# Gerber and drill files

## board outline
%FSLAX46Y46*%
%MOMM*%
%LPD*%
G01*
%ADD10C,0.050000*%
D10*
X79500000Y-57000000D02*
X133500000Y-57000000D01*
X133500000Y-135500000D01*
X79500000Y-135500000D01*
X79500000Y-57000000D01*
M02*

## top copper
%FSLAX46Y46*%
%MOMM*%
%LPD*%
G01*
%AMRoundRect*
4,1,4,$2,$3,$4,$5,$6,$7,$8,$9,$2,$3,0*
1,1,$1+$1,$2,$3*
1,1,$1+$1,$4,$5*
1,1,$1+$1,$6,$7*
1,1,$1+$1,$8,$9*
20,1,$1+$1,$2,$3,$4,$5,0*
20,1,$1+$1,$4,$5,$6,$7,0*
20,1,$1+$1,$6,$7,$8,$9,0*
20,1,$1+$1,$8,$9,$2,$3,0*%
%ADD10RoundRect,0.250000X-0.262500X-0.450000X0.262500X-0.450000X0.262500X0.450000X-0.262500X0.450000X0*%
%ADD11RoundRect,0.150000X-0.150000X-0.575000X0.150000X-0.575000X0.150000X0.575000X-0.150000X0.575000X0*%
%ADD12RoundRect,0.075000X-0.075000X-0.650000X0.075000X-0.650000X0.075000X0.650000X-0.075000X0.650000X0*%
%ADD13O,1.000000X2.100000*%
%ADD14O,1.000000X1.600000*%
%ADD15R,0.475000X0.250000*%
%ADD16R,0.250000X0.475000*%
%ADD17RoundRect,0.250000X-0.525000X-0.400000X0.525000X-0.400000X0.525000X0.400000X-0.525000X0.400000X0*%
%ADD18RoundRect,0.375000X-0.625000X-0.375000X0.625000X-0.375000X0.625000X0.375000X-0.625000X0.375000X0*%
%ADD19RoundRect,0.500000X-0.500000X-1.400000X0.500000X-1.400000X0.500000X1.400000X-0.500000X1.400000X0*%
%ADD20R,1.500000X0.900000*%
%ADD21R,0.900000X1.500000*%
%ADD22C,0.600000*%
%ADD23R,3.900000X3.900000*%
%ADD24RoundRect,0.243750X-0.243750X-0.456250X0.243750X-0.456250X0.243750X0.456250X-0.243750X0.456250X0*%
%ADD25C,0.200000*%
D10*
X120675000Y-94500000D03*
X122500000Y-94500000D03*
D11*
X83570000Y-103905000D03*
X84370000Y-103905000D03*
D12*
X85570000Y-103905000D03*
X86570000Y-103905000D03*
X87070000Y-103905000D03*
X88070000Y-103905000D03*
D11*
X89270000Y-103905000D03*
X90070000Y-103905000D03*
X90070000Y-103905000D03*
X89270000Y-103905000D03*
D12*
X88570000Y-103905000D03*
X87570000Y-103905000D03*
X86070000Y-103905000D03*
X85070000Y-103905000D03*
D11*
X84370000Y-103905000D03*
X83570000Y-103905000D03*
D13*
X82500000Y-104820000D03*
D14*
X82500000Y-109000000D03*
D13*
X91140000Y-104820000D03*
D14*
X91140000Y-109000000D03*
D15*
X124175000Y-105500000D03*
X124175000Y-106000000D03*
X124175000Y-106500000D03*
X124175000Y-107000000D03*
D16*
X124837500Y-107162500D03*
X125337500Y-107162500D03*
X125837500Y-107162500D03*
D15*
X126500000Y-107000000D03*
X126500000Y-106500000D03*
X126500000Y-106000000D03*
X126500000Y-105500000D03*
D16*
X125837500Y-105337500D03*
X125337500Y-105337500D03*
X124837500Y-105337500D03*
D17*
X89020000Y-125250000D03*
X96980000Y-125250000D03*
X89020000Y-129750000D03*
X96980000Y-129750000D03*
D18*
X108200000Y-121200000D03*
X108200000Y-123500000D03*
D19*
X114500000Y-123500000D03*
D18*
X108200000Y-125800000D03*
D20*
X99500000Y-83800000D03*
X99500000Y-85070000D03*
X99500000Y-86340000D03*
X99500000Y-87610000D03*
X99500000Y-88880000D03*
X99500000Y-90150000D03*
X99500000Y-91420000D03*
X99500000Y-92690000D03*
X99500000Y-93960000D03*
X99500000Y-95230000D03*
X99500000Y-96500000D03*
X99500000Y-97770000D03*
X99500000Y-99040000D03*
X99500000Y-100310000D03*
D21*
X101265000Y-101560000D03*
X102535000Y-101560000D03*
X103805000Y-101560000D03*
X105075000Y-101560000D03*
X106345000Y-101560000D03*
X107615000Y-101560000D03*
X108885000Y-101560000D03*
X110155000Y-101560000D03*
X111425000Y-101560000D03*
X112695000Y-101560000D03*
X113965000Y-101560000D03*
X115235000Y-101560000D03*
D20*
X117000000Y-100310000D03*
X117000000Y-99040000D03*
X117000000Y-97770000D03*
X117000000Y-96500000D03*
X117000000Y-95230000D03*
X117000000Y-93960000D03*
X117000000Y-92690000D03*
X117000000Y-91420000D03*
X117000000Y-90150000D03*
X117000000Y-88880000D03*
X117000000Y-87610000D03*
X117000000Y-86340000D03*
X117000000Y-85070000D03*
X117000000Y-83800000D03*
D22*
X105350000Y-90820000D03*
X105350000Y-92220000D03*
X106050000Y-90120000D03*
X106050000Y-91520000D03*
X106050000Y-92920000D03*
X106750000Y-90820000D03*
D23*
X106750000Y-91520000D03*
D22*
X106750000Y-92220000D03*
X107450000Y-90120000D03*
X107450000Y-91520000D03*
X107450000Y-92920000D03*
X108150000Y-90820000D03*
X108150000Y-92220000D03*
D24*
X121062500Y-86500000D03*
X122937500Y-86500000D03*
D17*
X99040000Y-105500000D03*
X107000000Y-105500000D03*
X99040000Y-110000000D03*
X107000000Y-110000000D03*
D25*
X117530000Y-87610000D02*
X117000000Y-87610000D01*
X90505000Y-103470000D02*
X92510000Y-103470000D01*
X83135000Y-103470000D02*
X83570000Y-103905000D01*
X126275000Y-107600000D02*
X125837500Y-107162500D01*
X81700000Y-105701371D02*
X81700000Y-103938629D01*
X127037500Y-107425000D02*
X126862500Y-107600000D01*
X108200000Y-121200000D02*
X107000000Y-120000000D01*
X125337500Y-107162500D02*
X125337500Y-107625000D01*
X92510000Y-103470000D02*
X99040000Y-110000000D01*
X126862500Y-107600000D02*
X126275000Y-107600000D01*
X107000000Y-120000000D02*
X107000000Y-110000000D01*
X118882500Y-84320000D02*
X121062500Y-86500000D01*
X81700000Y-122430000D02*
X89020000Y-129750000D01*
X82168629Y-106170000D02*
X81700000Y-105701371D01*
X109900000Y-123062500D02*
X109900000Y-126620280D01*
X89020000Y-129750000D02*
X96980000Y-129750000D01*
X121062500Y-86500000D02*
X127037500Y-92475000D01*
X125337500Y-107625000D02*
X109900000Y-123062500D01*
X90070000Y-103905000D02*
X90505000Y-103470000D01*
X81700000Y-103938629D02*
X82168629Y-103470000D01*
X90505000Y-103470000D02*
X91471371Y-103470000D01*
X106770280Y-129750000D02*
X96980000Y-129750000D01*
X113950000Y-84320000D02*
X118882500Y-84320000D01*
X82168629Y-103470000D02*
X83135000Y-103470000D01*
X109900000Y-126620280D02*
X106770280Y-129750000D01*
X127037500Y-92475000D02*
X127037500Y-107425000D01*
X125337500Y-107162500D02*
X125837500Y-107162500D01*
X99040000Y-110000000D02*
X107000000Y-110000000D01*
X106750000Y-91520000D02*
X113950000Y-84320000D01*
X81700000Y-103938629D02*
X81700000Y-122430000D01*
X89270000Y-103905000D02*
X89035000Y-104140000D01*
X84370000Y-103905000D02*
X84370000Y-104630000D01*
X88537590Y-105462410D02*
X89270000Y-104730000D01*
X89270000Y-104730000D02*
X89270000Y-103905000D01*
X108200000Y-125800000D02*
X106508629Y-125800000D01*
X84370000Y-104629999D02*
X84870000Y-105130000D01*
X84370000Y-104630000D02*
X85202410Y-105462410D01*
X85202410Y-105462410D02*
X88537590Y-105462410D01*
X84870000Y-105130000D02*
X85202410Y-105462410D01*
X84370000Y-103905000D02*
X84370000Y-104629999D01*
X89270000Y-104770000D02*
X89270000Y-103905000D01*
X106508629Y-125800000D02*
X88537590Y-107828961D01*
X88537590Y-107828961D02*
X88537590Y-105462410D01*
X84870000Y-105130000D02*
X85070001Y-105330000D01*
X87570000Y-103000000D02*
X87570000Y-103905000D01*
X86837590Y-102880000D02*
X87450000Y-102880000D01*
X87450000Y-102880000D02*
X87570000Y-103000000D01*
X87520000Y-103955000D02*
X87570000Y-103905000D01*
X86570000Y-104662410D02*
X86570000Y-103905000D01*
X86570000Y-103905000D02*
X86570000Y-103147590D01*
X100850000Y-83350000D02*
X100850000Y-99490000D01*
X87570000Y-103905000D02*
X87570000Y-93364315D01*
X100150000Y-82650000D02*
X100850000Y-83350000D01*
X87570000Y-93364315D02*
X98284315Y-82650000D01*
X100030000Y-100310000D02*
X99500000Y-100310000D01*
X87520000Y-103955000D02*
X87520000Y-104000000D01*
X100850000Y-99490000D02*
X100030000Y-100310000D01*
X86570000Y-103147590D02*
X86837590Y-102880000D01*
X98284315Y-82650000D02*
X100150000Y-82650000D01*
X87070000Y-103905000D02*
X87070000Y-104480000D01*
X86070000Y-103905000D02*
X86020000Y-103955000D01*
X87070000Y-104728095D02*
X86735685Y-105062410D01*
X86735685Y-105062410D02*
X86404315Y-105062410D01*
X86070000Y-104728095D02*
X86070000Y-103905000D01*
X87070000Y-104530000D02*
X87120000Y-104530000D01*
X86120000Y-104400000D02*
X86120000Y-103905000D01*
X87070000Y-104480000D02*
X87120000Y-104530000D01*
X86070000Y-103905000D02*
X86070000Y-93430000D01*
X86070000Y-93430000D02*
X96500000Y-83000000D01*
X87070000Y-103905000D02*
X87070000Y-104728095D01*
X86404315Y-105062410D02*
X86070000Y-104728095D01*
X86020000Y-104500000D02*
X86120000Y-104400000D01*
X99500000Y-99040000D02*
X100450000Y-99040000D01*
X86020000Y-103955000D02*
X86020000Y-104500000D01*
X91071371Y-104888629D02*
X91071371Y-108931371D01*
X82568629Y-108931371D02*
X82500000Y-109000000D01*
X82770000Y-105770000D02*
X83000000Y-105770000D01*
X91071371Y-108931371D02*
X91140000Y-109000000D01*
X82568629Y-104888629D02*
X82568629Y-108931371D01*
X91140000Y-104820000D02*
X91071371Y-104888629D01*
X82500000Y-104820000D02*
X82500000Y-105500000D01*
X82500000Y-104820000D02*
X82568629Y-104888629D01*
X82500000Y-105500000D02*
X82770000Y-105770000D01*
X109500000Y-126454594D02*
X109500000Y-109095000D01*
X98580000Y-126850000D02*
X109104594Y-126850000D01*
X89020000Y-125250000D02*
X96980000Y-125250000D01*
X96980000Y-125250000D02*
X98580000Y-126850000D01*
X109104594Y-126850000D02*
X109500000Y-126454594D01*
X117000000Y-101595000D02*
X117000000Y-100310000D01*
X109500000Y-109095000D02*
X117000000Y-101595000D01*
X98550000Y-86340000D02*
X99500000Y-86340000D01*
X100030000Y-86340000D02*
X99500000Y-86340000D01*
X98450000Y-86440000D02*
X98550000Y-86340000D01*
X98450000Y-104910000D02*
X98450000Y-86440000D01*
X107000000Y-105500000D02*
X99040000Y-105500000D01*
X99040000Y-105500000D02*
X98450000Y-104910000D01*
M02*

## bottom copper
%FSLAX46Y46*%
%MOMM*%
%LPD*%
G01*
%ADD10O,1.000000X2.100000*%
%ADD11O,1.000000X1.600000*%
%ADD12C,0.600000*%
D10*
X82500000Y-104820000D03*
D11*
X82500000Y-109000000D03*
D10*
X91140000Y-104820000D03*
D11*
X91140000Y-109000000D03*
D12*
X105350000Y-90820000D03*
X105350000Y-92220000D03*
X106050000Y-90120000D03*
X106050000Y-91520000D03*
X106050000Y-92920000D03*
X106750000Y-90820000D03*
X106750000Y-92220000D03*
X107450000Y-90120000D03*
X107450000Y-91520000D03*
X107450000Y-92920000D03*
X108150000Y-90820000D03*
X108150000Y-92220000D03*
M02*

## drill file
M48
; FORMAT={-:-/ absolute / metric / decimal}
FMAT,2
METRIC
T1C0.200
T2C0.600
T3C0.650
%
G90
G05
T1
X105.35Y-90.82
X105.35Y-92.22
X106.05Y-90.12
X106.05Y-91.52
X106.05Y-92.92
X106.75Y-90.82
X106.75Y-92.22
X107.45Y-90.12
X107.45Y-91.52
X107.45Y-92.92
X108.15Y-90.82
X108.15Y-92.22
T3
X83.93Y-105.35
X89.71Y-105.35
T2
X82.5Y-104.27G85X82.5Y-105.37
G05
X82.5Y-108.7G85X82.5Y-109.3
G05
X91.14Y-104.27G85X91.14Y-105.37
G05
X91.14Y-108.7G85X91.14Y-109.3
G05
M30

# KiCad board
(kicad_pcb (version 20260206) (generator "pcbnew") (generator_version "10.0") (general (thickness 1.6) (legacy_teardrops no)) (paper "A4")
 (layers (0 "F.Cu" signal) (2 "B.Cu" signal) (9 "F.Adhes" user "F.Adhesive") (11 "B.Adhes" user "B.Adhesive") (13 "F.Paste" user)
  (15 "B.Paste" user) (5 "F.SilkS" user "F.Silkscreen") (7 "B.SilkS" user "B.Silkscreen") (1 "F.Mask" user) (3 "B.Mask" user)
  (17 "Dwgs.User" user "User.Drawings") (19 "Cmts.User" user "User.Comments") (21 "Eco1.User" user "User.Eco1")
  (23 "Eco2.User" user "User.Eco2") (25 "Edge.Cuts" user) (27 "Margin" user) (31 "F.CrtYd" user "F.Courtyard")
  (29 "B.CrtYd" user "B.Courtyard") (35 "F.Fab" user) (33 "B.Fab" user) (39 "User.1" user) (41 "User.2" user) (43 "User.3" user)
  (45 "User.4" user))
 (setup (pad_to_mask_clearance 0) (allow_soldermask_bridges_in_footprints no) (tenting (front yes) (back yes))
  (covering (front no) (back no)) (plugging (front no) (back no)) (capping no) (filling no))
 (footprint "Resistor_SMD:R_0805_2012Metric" (layer "F.Cu") (at 121.5875 94.5)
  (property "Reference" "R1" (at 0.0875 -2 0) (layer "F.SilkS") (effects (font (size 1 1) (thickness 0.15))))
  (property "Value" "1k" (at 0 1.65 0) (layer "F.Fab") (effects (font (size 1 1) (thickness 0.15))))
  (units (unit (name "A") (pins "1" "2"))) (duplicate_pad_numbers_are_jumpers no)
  (pad "1" smd roundrect (at -0.9125 0) (size 1.025 1.4) (layers "F.Cu" "F.Mask" "F.Paste") (roundrect_rratio 0.243902) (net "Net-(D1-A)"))
  (pad "2" smd roundrect (at 0.9125 0) (size 1.025 1.4) (layers "F.Cu" "F.Mask" "F.Paste") (roundrect_rratio 0.243902) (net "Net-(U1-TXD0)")))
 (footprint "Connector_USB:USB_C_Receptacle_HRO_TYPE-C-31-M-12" (layer "F.Cu") (at 86.82 107.95)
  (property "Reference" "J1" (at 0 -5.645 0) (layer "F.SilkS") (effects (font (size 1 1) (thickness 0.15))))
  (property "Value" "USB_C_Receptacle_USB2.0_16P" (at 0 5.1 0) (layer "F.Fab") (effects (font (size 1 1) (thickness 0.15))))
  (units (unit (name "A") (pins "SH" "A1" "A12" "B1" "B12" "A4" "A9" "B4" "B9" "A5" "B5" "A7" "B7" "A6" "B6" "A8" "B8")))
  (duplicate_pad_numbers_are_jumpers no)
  (pad "" np_thru_hole circle (at -2.89 -2.6) (size 0.65 0.65) (drill 0.65) (layers "*.Cu" "*.Mask"))
  (pad "" np_thru_hole circle (at 2.89 -2.6) (size 0.65 0.65) (drill 0.65) (layers "*.Cu" "*.Mask"))
  (pad "A1" smd roundrect (at -3.25 -4.045) (size 0.6 1.45) (layers "F.Cu" "F.Mask" "F.Paste") (roundrect_rratio 0.25) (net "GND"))
  (pad "A4" smd roundrect (at -2.45 -4.045) (size 0.6 1.45) (layers "F.Cu" "F.Mask" "F.Paste") (roundrect_rratio 0.25) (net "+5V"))
  (pad "A5" smd roundrect (at -1.25 -4.045) (size 0.3 1.45) (layers "F.Cu" "F.Mask" "F.Paste") (roundrect_rratio 0.25)
   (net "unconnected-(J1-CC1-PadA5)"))
  (pad "A6" smd roundrect (at -0.25 -4.045) (size 0.3 1.45) (layers "F.Cu" "F.Mask" "F.Paste") (roundrect_rratio 0.25)
   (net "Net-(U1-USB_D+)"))
  (pad "A7" smd roundrect (at 0.25 -4.045) (size 0.3 1.45) (layers "F.Cu" "F.Mask" "F.Paste") (roundrect_rratio 0.25)
   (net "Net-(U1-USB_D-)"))
  (pad "A8" smd roundrect (at 1.25 -4.045) (size 0.3 1.45) (layers "F.Cu" "F.Mask" "F.Paste") (roundrect_rratio 0.25)
   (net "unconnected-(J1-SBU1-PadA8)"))
  (pad "A9" smd roundrect (at 2.45 -4.045) (size 0.6 1.45) (layers "F.Cu" "F.Mask" "F.Paste") (roundrect_rratio 0.25) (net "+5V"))
  (pad "A12" smd roundrect (at 3.25 -4.045) (size 0.6 1.45) (layers "F.Cu" "F.Mask" "F.Paste") (roundrect_rratio 0.25) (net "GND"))
  (pad "B1" smd roundrect (at 3.25 -4.045) (size 0.6 1.45) (layers "F.Cu" "F.Mask" "F.Paste") (roundrect_rratio 0.25) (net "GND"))
  (pad "B4" smd roundrect (at 2.45 -4.045) (size 0.6 1.45) (layers "F.Cu" "F.Mask" "F.Paste") (roundrect_rratio 0.25) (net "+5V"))
  (pad "B5" smd roundrect (at 1.75 -4.045) (size 0.3 1.45) (layers "F.Cu" "F.Mask" "F.Paste") (roundrect_rratio 0.25)
   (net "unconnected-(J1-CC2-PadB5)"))
  (pad "B6" smd roundrect (at 0.75 -4.045) (size 0.3 1.45) (layers "F.Cu" "F.Mask" "F.Paste") (roundrect_rratio 0.25)
   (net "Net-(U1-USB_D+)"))
  (pad "B7" smd roundrect (at -0.75 -4.045) (size 0.3 1.45) (layers "F.Cu" "F.Mask" "F.Paste") (roundrect_rratio 0.25)
   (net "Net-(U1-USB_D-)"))
  (pad "B8" smd roundrect (at -1.75 -4.045) (size 0.3 1.45) (layers "F.Cu" "F.Mask" "F.Paste") (roundrect_rratio 0.25)
   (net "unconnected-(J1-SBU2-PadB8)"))
  (pad "B9" smd roundrect (at -2.45 -4.045) (size 0.6 1.45) (layers "F.Cu" "F.Mask" "F.Paste") (roundrect_rratio 0.25) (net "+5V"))
  (pad "B12" smd roundrect (at -3.25 -4.045) (size 0.6 1.45) (layers "F.Cu" "F.Mask" "F.Paste") (roundrect_rratio 0.25) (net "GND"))
  (pad "SH" thru_hole oval (at -4.32 -3.13) (size 1 2.1) (drill oval 0.6 1.7) (layers "*.Cu" "*.Mask") (remove_unused_layers no)
   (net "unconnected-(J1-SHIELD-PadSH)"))
  (pad "SH" thru_hole oval (at -4.32 1.05) (size 1 1.6) (drill oval 0.6 1.2) (layers "*.Cu" "*.Mask") (remove_unused_layers no)
   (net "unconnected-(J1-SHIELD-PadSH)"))
  (pad "SH" thru_hole oval (at 4.32 -3.13) (size 1 2.1) (drill oval 0.6 1.7) (layers "*.Cu" "*.Mask") (remove_unused_layers no)
   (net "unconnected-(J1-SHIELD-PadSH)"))
  (pad "SH" thru_hole oval (at 4.32 1.05) (size 1 1.6) (drill oval 0.6 1.2) (layers "*.Cu" "*.Mask") (remove_unused_layers no)
   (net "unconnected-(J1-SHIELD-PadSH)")))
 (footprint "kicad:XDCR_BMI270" (layer "F.Cu") (at 125.3375 106.25)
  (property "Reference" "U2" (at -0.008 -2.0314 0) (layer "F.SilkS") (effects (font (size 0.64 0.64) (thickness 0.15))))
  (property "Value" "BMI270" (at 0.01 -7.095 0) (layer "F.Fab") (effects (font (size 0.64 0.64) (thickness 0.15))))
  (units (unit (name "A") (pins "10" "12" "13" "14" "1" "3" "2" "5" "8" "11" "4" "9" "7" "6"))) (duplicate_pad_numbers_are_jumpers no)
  (pad "1" smd rect (at -1.1625 -0.75) (size 0.475 0.25) (layers "F.Cu" "F.Mask" "F.Paste") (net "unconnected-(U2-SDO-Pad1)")
   (solder_mask_margin 0.102))
  (pad "2" smd rect (at -1.1625 -0.25) (size 0.475 0.25) (layers "F.Cu" "F.Mask" "F.Paste") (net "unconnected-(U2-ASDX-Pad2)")
   (solder_mask_margin 0.102))
  (pad "3" smd rect (at -1.1625 0.25) (size 0.475 0.25) (layers "F.Cu" "F.Mask" "F.Paste") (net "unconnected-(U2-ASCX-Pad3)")
   (solder_mask_margin 0.102))
  (pad "4" smd rect (at -1.1625 0.75) (size 0.475 0.25) (layers "F.Cu" "F.Mask" "F.Paste") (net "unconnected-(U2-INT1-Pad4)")
   (solder_mask_margin 0.102))
  (pad "5" smd rect (at -0.5 0.9125) (size 0.25 0.475) (layers "F.Cu" "F.Mask" "F.Paste") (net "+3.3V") (solder_mask_margin 0.102))
  (pad "6" smd rect (at 0 0.9125) (size 0.25 0.475) (layers "F.Cu" "F.Mask" "F.Paste") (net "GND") (solder_mask_margin 0.102))
  (pad "7" smd rect (at 0.5 0.9125) (size 0.25 0.475) (layers "F.Cu" "F.Mask" "F.Paste") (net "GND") (solder_mask_margin 0.102))
  (pad "8" smd rect (at 1.1625 0.75) (size 0.475 0.25) (layers "F.Cu" "F.Mask" "F.Paste") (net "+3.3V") (solder_mask_margin 0.102))
  (pad "9" smd rect (at 1.1625 0.25) (size 0.475 0.25) (layers "F.Cu" "F.Mask" "F.Paste") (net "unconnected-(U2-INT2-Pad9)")
   (solder_mask_margin 0.102))
  (pad "10" smd rect (at 1.1625 -0.25) (size 0.475 0.25) (layers "F.Cu" "F.Mask" "F.Paste") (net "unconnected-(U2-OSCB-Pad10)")
   (solder_mask_margin 0.102))
  (pad "11" smd rect (at 1.1625 -0.75) (size 0.475 0.25) (layers "F.Cu" "F.Mask" "F.Paste") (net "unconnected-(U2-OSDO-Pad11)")
   (solder_mask_margin 0.102))
  (pad "12" smd rect (at 0.5 -0.9125) (size 0.25 0.475) (layers "F.Cu" "F.Mask" "F.Paste") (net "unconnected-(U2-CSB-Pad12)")
   (solder_mask_margin 0.102))
  (pad "13" smd rect (at 0 -0.9125) (size 0.25 0.475) (layers "F.Cu" "F.Mask" "F.Paste") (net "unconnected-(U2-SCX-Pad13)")
   (solder_mask_margin 0.102))
  (pad "14" smd rect (at -0.5 -0.9125) (size 0.25 0.475) (layers "F.Cu" "F.Mask" "F.Paste") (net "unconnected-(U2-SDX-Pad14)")
   (solder_mask_margin 0.102)))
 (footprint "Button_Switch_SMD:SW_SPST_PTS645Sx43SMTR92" (layer "F.Cu") (at 93 127.5)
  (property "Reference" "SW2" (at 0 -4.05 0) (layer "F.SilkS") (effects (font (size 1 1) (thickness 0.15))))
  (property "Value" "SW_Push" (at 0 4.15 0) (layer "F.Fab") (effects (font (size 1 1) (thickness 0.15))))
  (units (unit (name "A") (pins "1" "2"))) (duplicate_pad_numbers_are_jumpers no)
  (pad "1" smd roundrect (at -3.98 -2.25) (size 1.55 1.3) (layers "F.Cu" "F.Mask" "F.Paste") (roundrect_rratio 0.1923076923)
   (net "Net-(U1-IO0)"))
  (pad "1" smd roundrect (at 3.98 -2.25) (size 1.55 1.3) (layers "F.Cu" "F.Mask" "F.Paste") (roundrect_rratio 0.1923076923)
   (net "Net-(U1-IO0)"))
  (pad "2" smd roundrect (at -3.98 2.25) (size 1.55 1.3) (layers "F.Cu" "F.Mask" "F.Paste") (roundrect_rratio 0.1923076923) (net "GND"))
  (pad "2" smd roundrect (at 3.98 2.25) (size 1.55 1.3) (layers "F.Cu" "F.Mask" "F.Paste") (roundrect_rratio 0.1923076923) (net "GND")))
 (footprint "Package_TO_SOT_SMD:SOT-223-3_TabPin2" (layer "F.Cu") (at 111.35 123.5)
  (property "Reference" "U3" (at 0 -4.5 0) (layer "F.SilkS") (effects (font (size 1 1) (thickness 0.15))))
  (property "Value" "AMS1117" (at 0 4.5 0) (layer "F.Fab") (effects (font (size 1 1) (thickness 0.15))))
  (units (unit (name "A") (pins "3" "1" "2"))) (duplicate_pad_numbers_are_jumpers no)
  (pad "1" smd roundrect (at -3.15 -2.3) (size 2 1.5) (layers "F.Cu" "F.Mask" "F.Paste") (roundrect_rratio 0.25) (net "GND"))
  (pad "2" smd roundrect (at -3.15 0) (size 2 1.5) (layers "F.Cu" "F.Mask" "F.Paste") (roundrect_rratio 0.25) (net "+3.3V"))
  (pad "2" smd roundrect (at 3.15 0) (size 2 3.8) (layers "F.Cu" "F.Mask" "F.Paste") (roundrect_rratio 0.25) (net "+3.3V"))
  (pad "3" smd roundrect (at -3.15 2.3) (size 2 1.5) (layers "F.Cu" "F.Mask" "F.Paste") (roundrect_rratio 0.25) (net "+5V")))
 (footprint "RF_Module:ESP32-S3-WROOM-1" (layer "F.Cu") (at 108.25 89.06)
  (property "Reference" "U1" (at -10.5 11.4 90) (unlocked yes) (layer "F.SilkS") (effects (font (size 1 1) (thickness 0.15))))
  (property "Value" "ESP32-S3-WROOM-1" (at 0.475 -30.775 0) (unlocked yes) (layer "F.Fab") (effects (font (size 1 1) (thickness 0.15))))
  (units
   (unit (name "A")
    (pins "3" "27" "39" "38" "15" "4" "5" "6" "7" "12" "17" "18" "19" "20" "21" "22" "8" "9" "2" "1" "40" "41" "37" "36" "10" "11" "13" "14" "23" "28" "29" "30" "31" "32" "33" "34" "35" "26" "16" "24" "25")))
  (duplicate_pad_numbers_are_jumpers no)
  (pad "" smd rect (at -2.9 1.06) (size 0.9 0.9) (layers "F.Paste"))
  (pad "" smd rect (at -2.9 2.46 270) (size 0.9 0.9) (layers "F.Paste"))
  (pad "" smd rect (at -2.9 3.86) (size 0.9 0.9) (layers "F.Paste"))
  (pad "" smd rect (at -1.5 1.06 270) (size 0.9 0.9) (layers "F.Paste"))
  (pad "" smd rect (at -1.5 2.46 270) (size 0.9 0.9) (layers "F.Paste"))
  (pad "" smd rect (at -1.5 3.86 270) (size 0.9 0.9) (layers "F.Paste"))
  (pad "" smd rect (at -0.1 1.06 270) (size 0.9 0.9) (layers "F.Paste"))
  (pad "" smd rect (at -0.1 2.46 270) (size 0.9 0.9) (layers "F.Paste"))
  (pad "" smd rect (at -0.1 3.86 270) (size 0.9 0.9) (layers "F.Paste"))
  (pad "1" smd rect (at -8.75 -5.26) (size 1.5 0.9) (layers "F.Cu" "F.Mask" "F.Paste") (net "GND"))
  (pad "2" smd rect (at -8.75 -3.99) (size 1.5 0.9) (layers "F.Cu" "F.Mask" "F.Paste") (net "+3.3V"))
  (pad "3" smd rect (at -8.75 -2.72) (size 1.5 0.9) (layers "F.Cu" "F.Mask" "F.Paste") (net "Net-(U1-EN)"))
  (pad "4" smd rect (at -8.75 -1.45) (size 1.5 0.9) (layers "F.Cu" "F.Mask" "F.Paste") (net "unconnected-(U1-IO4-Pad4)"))
  (pad "5" smd rect (at -8.75 -0.18) (size 1.5 0.9) (layers "F.Cu" "F.Mask" "F.Paste") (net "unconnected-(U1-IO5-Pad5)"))
  (pad "6" smd rect (at -8.75 1.09) (size 1.5 0.9) (layers "F.Cu" "F.Mask" "F.Paste") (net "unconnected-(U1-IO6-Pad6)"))
  (pad "7" smd rect (at -8.75 2.36) (size 1.5 0.9) (layers "F.Cu" "F.Mask" "F.Paste") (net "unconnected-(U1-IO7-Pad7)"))
  (pad "8" smd rect (at -8.75 3.63) (size 1.5 0.9) (layers "F.Cu" "F.Mask" "F.Paste") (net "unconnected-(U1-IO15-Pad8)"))
  (pad "9" smd rect (at -8.75 4.9) (size 1.5 0.9) (layers "F.Cu" "F.Mask" "F.Paste") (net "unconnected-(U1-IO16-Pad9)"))
  (pad "10" smd rect (at -8.75 6.17) (size 1.5 0.9) (layers "F.Cu" "F.Mask" "F.Paste") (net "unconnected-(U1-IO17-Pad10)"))
  (pad "11" smd rect (at -8.75 7.44) (size 1.5 0.9) (layers "F.Cu" "F.Mask" "F.Paste") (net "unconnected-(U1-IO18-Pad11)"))
  (pad "12" smd rect (at -8.75 8.71) (size 1.5 0.9) (layers "F.Cu" "F.Mask" "F.Paste") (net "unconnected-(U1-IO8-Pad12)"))
  (pad "13" smd rect (at -8.75 9.98) (size 1.5 0.9) (layers "F.Cu" "F.Mask" "F.Paste") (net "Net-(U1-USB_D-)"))
  (pad "14" smd rect (at -8.75 11.25 180) (size 1.5 0.9) (layers "F.Cu" "F.Mask" "F.Paste") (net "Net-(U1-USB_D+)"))
  (pad "15" smd rect (at -6.985 12.5 270) (size 1.5 0.9) (layers "F.Cu" "F.Mask" "F.Paste") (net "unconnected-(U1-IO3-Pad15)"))
  (pad "16" smd rect (at -5.715 12.5 270) (size 1.5 0.9) (layers "F.Cu" "F.Mask" "F.Paste") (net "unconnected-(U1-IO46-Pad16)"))
  (pad "17" smd rect (at -4.445 12.5 270) (size 1.5 0.9) (layers "F.Cu" "F.Mask" "F.Paste") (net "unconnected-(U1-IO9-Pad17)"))
  (pad "18" smd rect (at -3.175 12.5 270) (size 1.5 0.9) (layers "F.Cu" "F.Mask" "F.Paste") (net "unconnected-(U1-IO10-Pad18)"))
  (pad "19" smd rect (at -1.905 12.5 270) (size 1.5 0.9) (layers "F.Cu" "F.Mask" "F.Paste") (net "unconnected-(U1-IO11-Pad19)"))
  (pad "20" smd rect (at -0.635 12.5 270) (size 1.5 0.9) (layers "F.Cu" "F.Mask" "F.Paste") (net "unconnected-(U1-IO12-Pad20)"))
  (pad "21" smd rect (at 0.635 12.5 270) (size 1.5 0.9) (layers "F.Cu" "F.Mask" "F.Paste") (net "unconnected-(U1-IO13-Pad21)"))
  (pad "22" smd rect (at 1.905 12.5 270) (size 1.5 0.9) (layers "F.Cu" "F.Mask" "F.Paste") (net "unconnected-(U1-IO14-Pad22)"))
  (pad "23" smd rect (at 3.175 12.5 270) (size 1.5 0.9) (layers "F.Cu" "F.Mask" "F.Paste") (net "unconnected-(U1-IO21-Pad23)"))
  (pad "24" smd rect (at 4.445 12.5 270) (size 1.5 0.9) (layers "F.Cu" "F.Mask" "F.Paste") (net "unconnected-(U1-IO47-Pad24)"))
  (pad "25" smd rect (at 5.715 12.5 270) (size 1.5 0.9) (layers "F.Cu" "F.Mask" "F.Paste") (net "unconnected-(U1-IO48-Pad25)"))
  (pad "26" smd rect (at 6.985 12.5 270) (size 1.5 0.9) (layers "F.Cu" "F.Mask" "F.Paste") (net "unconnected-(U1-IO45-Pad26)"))
  (pad "27" smd rect (at 8.75 11.25) (size 1.5 0.9) (layers "F.Cu" "F.Mask" "F.Paste") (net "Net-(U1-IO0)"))
  (pad "28" smd rect (at 8.75 9.98) (size 1.5 0.9) (layers "F.Cu" "F.Mask" "F.Paste") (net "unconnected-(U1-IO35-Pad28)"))
  (pad "29" smd rect (at 8.75 8.71) (size 1.5 0.9) (layers "F.Cu" "F.Mask" "F.Paste") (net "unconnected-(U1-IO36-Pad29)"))
  (pad "30" smd rect (at 8.75 7.44) (size 1.5 0.9) (layers "F.Cu" "F.Mask" "F.Paste") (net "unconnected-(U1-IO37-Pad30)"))
  (pad "31" smd rect (at 8.75 6.17) (size 1.5 0.9) (layers "F.Cu" "F.Mask" "F.Paste") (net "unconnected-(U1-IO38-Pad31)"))
  (pad "32" smd rect (at 8.75 4.9) (size 1.5 0.9) (layers "F.Cu" "F.Mask" "F.Paste") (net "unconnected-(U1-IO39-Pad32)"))
  (pad "33" smd rect (at 8.75 3.63) (size 1.5 0.9) (layers "F.Cu" "F.Mask" "F.Paste") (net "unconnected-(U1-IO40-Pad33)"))
  (pad "34" smd rect (at 8.75 2.36) (size 1.5 0.9) (layers "F.Cu" "F.Mask" "F.Paste") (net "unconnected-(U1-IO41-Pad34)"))
  (pad "35" smd rect (at 8.75 1.09) (size 1.5 0.9) (layers "F.Cu" "F.Mask" "F.Paste") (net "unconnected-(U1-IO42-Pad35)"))
  (pad "36" smd rect (at 8.75 -0.18) (size 1.5 0.9) (layers "F.Cu" "F.Mask" "F.Paste") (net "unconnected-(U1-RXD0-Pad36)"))
  (pad "37" smd rect (at 8.75 -1.45) (size 1.5 0.9) (layers "F.Cu" "F.Mask" "F.Paste") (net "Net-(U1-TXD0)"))
  (pad "38" smd rect (at 8.75 -2.72) (size 1.5 0.9) (layers "F.Cu" "F.Mask" "F.Paste") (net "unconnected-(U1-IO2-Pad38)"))
  (pad "39" smd rect (at 8.75 -3.99) (size 1.5 0.9) (layers "F.Cu" "F.Mask" "F.Paste") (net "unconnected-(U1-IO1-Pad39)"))
  (pad "40" smd rect (at 8.75 -5.26) (size 1.5 0.9) (layers "F.Cu" "F.Mask" "F.Paste") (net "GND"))
  (pad "41" thru_hole circle (at -2.9 1.76 90) (size 0.6 0.6) (drill 0.2) (layers "*.Cu" "F.Mask") (remove_unused_layers no) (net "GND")
   (zone_connect 2))
  (pad "41" thru_hole circle (at -2.9 3.16) (size 0.6 0.6) (drill 0.2) (layers "*.Cu" "F.Mask") (remove_unused_layers no) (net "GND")
   (zone_connect 2))
  (pad "41" thru_hole circle (at -2.2 1.06) (size 0.6 0.6) (drill 0.2) (layers "*.Cu" "F.Mask") (remove_unused_layers no) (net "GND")
   (zone_connect 2))
  (pad "41" thru_hole circle (at -2.2 2.46) (size 0.6 0.6) (drill 0.2) (layers "*.Cu" "F.Mask") (remove_unused_layers no) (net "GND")
   (zone_connect 2))
  (pad "41" thru_hole circle (at -2.2 3.86) (size 0.6 0.6) (drill 0.2) (layers "*.Cu" "F.Mask") (remove_unused_layers no) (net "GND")
   (zone_connect 2))
  (pad "41" thru_hole circle (at -1.5 1.76) (size 0.6 0.6) (drill 0.2) (layers "*.Cu" "F.Mask") (remove_unused_layers no) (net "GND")
   (zone_connect 2))
  (pad "41" smd rect (at -1.5 2.46 270) (size 3.9 3.9) (layers "F.Cu" "F.Mask") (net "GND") (zone_connect 2))
  (pad "41" thru_hole circle (at -1.5 3.16) (size 0.6 0.6) (drill 0.2) (layers "*.Cu" "F.Mask") (remove_unused_layers no) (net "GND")
   (zone_connect 2))
  (pad "41" thru_hole circle (at -0.8 1.06) (size 0.6 0.6) (drill 0.2) (layers "*.Cu" "F.Mask") (remove_unused_layers no) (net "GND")
   (zone_connect 2))
  (pad "41" thru_hole circle (at -0.8 2.46) (size 0.6 0.6) (drill 0.2) (layers "*.Cu" "F.Mask") (remove_unused_layers no) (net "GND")
   (zone_connect 2))
  (pad "41" thru_hole circle (at -0.8 3.86) (size 0.6 0.6) (drill 0.2) (layers "*.Cu" "F.Mask") (remove_unused_layers no) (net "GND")
   (zone_connect 2))
  (pad "41" thru_hole circle (at -0.1 1.76) (size 0.6 0.6) (drill 0.2) (layers "*.Cu" "F.Mask") (remove_unused_layers no) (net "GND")
   (zone_connect 2))
  (pad "41" thru_hole circle (at -0.1 3.16) (size 0.6 0.6) (drill 0.2) (layers "*.Cu" "F.Mask") (remove_unused_layers no) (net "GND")
   (zone_connect 2))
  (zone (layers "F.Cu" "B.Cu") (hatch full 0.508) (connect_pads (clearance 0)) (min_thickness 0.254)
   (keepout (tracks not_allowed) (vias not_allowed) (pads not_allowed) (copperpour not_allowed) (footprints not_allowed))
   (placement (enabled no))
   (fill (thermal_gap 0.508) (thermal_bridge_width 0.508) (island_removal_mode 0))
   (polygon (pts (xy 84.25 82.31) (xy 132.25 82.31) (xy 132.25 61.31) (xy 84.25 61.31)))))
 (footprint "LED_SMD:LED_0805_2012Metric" (layer "F.Cu") (at 122 86.5)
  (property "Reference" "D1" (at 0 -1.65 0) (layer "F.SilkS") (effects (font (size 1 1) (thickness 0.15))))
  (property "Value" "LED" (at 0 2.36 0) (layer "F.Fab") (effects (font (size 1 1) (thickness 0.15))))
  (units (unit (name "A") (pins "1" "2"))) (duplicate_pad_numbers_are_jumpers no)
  (pad "1" smd roundrect (at -0.9375 0) (size 0.975 1.4) (layers "F.Cu" "F.Mask" "F.Paste") (roundrect_rratio 0.25) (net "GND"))
  (pad "2" smd roundrect (at 0.9375 0) (size 0.975 1.4) (layers "F.Cu" "F.Mask" "F.Paste") (roundrect_rratio 0.25) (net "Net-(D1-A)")))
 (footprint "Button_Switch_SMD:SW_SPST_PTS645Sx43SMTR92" (layer "F.Cu") (at 103.02 107.75)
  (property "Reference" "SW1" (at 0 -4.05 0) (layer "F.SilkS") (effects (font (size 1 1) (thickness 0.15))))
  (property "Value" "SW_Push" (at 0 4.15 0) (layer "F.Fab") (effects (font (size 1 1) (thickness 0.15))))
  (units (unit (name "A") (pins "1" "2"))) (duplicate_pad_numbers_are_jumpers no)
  (pad "1" smd roundrect (at -3.98 -2.25) (size 1.55 1.3) (layers "F.Cu" "F.Mask" "F.Paste") (roundrect_rratio 0.1923076923)
   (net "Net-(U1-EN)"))
  (pad "1" smd roundrect (at 3.98 -2.25) (size 1.55 1.3) (layers "F.Cu" "F.Mask" "F.Paste") (roundrect_rratio 0.1923076923)
   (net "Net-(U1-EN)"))
  (pad "2" smd roundrect (at -3.98 2.25) (size 1.55 1.3) (layers "F.Cu" "F.Mask" "F.Paste") (roundrect_rratio 0.1923076923) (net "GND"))
  (pad "2" smd roundrect (at 3.98 2.25) (size 1.55 1.3) (layers "F.Cu" "F.Mask" "F.Paste") (roundrect_rratio 0.1923076923) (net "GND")))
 (gr_rect (start 79.5 57) (end 133.5 135.5) (stroke (width 0.05) (type default)) (fill no) (layer "Edge.Cuts"))
 (segment (start 117.53 87.61) (end 117 87.61) (width 0.2) (layer "F.Cu") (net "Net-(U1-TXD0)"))
 (segment (start 90.505 103.47) (end 92.51 103.47) (width 0.2) (layer "F.Cu") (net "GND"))
 (segment (start 83.135 103.47) (end 83.57 103.905) (width 0.2) (layer "F.Cu") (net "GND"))
 (segment (start 126.275 107.6) (end 125.8375 107.1625) (width 0.2) (layer "F.Cu") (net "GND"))
 (segment (start 81.7 105.701371) (end 81.7 103.938629) (width 0.2) (layer "F.Cu") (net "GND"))
 (segment (start 127.0375 107.425) (end 126.8625 107.6) (width 0.2) (layer "F.Cu") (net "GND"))
 (segment (start 108.2 121.2) (end 107 120) (width 0.2) (layer "F.Cu") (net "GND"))
 (segment (start 125.3375 107.1625) (end 125.3375 107.625) (width 0.2) (layer "F.Cu") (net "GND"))
 (segment (start 92.51 103.47) (end 99.04 110) (width 0.2) (layer "F.Cu") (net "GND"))
 (segment (start 126.8625 107.6) (end 126.275 107.6) (width 0.2) (layer "F.Cu") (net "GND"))
 (segment (start 107 120) (end 107 110) (width 0.2) (layer "F.Cu") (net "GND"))
 (segment (start 118.8825 84.32) (end 121.0625 86.5) (width 0.2) (layer "F.Cu") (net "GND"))
 (segment (start 81.7 122.43) (end 89.02 129.75) (width 0.2) (layer "F.Cu") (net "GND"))
 (segment (start 82.168629 106.17) (end 81.7 105.701371) (width 0.2) (layer "F.Cu") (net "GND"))
 (segment (start 109.9 123.0625) (end 109.9 126.62028) (width 0.2) (layer "F.Cu") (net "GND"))
 (segment (start 89.02 129.75) (end 96.98 129.75) (width 0.2) (layer "F.Cu") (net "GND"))
 (segment (start 121.0625 86.5) (end 127.0375 92.475) (width 0.2) (layer "F.Cu") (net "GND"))
 (segment (start 125.3375 107.625) (end 109.9 123.0625) (width 0.2) (layer "F.Cu") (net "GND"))
 (segment (start 90.07 103.905) (end 90.505 103.47) (width 0.2) (layer "F.Cu") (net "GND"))
 (segment (start 81.7 103.938629) (end 82.168629 103.47) (width 0.2) (layer "F.Cu") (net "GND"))
 (segment (start 90.505 103.47) (end 91.471371 103.47) (width 0.2) (layer "F.Cu") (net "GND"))
 (segment (start 106.77028 129.75) (end 96.98 129.75) (width 0.2) (layer "F.Cu") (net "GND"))
 (segment (start 113.95 84.32) (end 118.8825 84.32) (width 0.2) (layer "F.Cu") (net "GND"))
 (segment (start 82.168629 103.47) (end 83.135 103.47) (width 0.2) (layer "F.Cu") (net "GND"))
 (segment (start 109.9 126.62028) (end 106.77028 129.75) (width 0.2) (layer "F.Cu") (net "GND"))
 (segment (start 127.0375 92.475) (end 127.0375 107.425) (width 0.2) (layer "F.Cu") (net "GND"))
 (segment (start 125.3375 107.1625) (end 125.8375 107.1625) (width 0.2) (layer "F.Cu") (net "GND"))
 (segment (start 99.04 110) (end 107 110) (width 0.2) (layer "F.Cu") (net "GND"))
 (segment (start 106.75 91.52) (end 113.95 84.32) (width 0.2) (layer "F.Cu") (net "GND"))
 (segment (start 81.7 103.938629) (end 81.7 122.43) (width 0.2) (layer "F.Cu") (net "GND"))
 (segment (start 89.27 103.905) (end 89.035 104.14) (width 0.2) (layer "F.Cu") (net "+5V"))
 (segment (start 84.37 103.905) (end 84.37 104.63) (width 0.2) (layer "F.Cu") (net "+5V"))
 (segment (start 88.53759 105.46241) (end 89.27 104.73) (width 0.2) (layer "F.Cu") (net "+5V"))
 (segment (start 89.27 104.73) (end 89.27 103.905) (width 0.2) (layer "F.Cu") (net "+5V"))
 (segment (start 108.2 125.8) (end 106.508629 125.8) (width 0.2) (layer "F.Cu") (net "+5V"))
 (segment (start 84.37 104.629999) (end 84.87 105.13) (width 0.2) (layer "F.Cu") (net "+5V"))
 (segment (start 84.37 104.63) (end 85.20241 105.46241) (width 0.2) (layer "F.Cu") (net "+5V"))
 (segment (start 85.20241 105.46241) (end 88.53759 105.46241) (width 0.2) (layer "F.Cu") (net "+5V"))
 (segment (start 84.87 105.13) (end 85.20241 105.46241) (width 0.2) (layer "F.Cu") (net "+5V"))
 (segment (start 84.37 103.905) (end 84.37 104.629999) (width 0.2) (layer "F.Cu") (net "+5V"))
 (segment (start 89.27 104.77) (end 89.27 103.905) (width 0.2) (layer "F.Cu") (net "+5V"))
 (segment (start 106.508629 125.8) (end 88.53759 107.828961) (width 0.2) (layer "F.Cu") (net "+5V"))
 (segment (start 88.53759 107.828961) (end 88.53759 105.46241) (width 0.2) (layer "F.Cu") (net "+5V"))
 (segment (start 84.87 105.13) (end 85.070001 105.33) (width 0.2) (layer "F.Cu") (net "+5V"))
 (segment (start 87.57 103) (end 87.57 103.905) (width 0.2) (layer "F.Cu") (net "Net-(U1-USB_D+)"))
 (segment (start 86.83759 102.88) (end 87.45 102.88) (width 0.2) (layer "F.Cu") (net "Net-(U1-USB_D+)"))
 (segment (start 87.45 102.88) (end 87.57 103) (width 0.2) (layer "F.Cu") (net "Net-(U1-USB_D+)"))
 (segment (start 87.52 103.955) (end 87.57 103.905) (width 0.2) (layer "F.Cu") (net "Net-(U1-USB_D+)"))
 (segment (start 86.57 104.66241) (end 86.57 103.905) (width 0.2) (layer "F.Cu") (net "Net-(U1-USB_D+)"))
 (segment (start 86.57 103.905) (end 86.57 103.14759) (width 0.2) (layer "F.Cu") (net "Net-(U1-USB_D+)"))
 (segment (start 100.85 83.35) (end 100.85 99.49) (width 0.2) (layer "F.Cu") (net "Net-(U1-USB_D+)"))
 (segment (start 87.57 103.905) (end 87.57 93.364315) (width 0.2) (layer "F.Cu") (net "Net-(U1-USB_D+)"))
 (segment (start 100.15 82.65) (end 100.85 83.35) (width 0.2) (layer "F.Cu") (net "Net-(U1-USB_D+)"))
 (segment (start 87.57 93.364315) (end 98.284315 82.65) (width 0.2) (layer "F.Cu") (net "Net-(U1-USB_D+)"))
 (segment (start 100.03 100.31) (end 99.5 100.31) (width 0.2) (layer "F.Cu") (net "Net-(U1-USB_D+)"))
 (segment (start 87.52 103.955) (end 87.52 104) (width 0.2) (layer "F.Cu") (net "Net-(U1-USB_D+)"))
 (segment (start 100.85 99.49) (end 100.03 100.31) (width 0.2) (layer "F.Cu") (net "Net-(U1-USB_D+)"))
 (segment (start 86.57 103.14759) (end 86.83759 102.88) (width 0.2) (layer "F.Cu") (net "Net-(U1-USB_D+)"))
 (segment (start 98.284315 82.65) (end 100.15 82.65) (width 0.2) (layer "F.Cu") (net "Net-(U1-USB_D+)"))
 (segment (start 87.07 103.905) (end 87.07 104.48) (width 0.2) (layer "F.Cu") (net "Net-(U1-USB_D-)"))
 (segment (start 86.07 103.905) (end 86.02 103.955) (width 0.2) (layer "F.Cu") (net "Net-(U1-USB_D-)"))
 (segment (start 87.07 104.728095) (end 86.735685 105.06241) (width 0.2) (layer "F.Cu") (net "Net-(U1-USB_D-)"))
 (segment (start 86.735685 105.06241) (end 86.404315 105.06241) (width 0.2) (layer "F.Cu") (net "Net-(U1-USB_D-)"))
 (segment (start 86.07 104.728095) (end 86.07 103.905) (width 0.2) (layer "F.Cu") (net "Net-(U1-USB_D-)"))
 (segment (start 87.07 104.53) (end 87.12 104.53) (width 0.2) (layer "F.Cu") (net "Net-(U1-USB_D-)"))
 (segment (start 86.12 104.4) (end 86.12 103.905) (width 0.2) (layer "F.Cu") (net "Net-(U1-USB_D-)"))
 (segment (start 87.07 104.48) (end 87.12 104.53) (width 0.2) (layer "F.Cu") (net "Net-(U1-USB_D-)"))
 (segment (start 86.07 103.905) (end 86.07 93.43) (width 0.2) (layer "F.Cu") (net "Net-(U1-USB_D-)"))
 (segment (start 86.07 93.43) (end 96.5 83) (width 0.2) (layer "F.Cu") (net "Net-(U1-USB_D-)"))
 (segment (start 87.07 103.905) (end 87.07 104.728095) (width 0.2) (layer "F.Cu") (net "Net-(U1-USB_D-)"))
 (segment (start 86.404315 105.06241) (end 86.07 104.728095) (width 0.2) (layer "F.Cu") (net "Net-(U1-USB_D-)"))
 (segment (start 86.02 104.5) (end 86.12 104.4) (width 0.2) (layer "F.Cu") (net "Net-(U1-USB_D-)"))
 (segment (start 99.5 99.04) (end 100.45 99.04) (width 0.2) (layer "F.Cu") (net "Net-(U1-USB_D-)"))
 (segment (start 86.02 103.955) (end 86.02 104.5) (width 0.2) (layer "F.Cu") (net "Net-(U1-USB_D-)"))
 (segment (start 91.071371 104.888629) (end 91.071371 108.931371) (width 0.2) (layer "F.Cu") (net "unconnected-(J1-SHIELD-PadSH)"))
 (segment (start 82.568629 108.931371) (end 82.5 109) (width 0.2) (layer "F.Cu") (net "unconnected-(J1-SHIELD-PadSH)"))
 (segment (start 82.77 105.77) (end 83 105.77) (width 0.2) (layer "F.Cu") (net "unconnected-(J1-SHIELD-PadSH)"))
 (segment (start 91.071371 108.931371) (end 91.14 109) (width 0.2) (layer "F.Cu") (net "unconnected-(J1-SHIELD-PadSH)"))
 (segment (start 82.568629 104.888629) (end 82.568629 108.931371) (width 0.2) (layer "F.Cu") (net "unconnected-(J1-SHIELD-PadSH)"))
 (segment (start 91.14 104.82) (end 91.071371 104.888629) (width 0.2) (layer "F.Cu") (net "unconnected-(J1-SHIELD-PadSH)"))
 (segment (start 82.5 104.82) (end 82.5 105.5) (width 0.2) (layer "F.Cu") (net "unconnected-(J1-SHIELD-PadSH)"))
 (segment (start 82.5 104.82) (end 82.568629 104.888629) (width 0.2) (layer "F.Cu") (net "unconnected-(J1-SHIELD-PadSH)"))
 (segment (start 82.5 105.5) (end 82.77 105.77) (width 0.2) (layer "F.Cu") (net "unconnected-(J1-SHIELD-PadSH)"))
 (segment (start 109.5 126.454594) (end 109.5 109.095) (width 0.2) (layer "F.Cu") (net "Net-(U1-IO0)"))
 (segment (start 98.58 126.85) (end 109.104594 126.85) (width 0.2) (layer "F.Cu") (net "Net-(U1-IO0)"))
 (segment (start 89.02 125.25) (end 96.98 125.25) (width 0.2) (layer "F.Cu") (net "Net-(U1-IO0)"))
 (segment (start 96.98 125.25) (end 98.58 126.85) (width 0.2) (layer "F.Cu") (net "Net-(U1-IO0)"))
 (segment (start 109.104594 126.85) (end 109.5 126.454594) (width 0.2) (layer "F.Cu") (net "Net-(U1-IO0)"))
 (segment (start 117 101.595) (end 117 100.31) (width 0.2) (layer "F.Cu") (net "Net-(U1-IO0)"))
 (segment (start 109.5 109.095) (end 117 101.595) (width 0.2) (layer "F.Cu") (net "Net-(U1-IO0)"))
 (segment (start 98.55 86.34) (end 99.5 86.34) (width 0.2) (layer "F.Cu") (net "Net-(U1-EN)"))
 (segment (start 100.03 86.34) (end 99.5 86.34) (width 0.2) (layer "F.Cu") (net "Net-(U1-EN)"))
 (segment (start 98.45 86.44) (end 98.55 86.34) (width 0.2) (layer "F.Cu") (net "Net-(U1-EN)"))
 (segment (start 98.45 104.91) (end 98.45 86.44) (width 0.2) (layer "F.Cu") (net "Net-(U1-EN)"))
 (segment (start 107 105.5) (end 99.04 105.5) (width 0.2) (layer "F.Cu") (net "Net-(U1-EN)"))
 (segment (start 99.04 105.5) (end 98.45 104.91) (width 0.2) (layer "F.Cu") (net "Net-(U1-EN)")))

